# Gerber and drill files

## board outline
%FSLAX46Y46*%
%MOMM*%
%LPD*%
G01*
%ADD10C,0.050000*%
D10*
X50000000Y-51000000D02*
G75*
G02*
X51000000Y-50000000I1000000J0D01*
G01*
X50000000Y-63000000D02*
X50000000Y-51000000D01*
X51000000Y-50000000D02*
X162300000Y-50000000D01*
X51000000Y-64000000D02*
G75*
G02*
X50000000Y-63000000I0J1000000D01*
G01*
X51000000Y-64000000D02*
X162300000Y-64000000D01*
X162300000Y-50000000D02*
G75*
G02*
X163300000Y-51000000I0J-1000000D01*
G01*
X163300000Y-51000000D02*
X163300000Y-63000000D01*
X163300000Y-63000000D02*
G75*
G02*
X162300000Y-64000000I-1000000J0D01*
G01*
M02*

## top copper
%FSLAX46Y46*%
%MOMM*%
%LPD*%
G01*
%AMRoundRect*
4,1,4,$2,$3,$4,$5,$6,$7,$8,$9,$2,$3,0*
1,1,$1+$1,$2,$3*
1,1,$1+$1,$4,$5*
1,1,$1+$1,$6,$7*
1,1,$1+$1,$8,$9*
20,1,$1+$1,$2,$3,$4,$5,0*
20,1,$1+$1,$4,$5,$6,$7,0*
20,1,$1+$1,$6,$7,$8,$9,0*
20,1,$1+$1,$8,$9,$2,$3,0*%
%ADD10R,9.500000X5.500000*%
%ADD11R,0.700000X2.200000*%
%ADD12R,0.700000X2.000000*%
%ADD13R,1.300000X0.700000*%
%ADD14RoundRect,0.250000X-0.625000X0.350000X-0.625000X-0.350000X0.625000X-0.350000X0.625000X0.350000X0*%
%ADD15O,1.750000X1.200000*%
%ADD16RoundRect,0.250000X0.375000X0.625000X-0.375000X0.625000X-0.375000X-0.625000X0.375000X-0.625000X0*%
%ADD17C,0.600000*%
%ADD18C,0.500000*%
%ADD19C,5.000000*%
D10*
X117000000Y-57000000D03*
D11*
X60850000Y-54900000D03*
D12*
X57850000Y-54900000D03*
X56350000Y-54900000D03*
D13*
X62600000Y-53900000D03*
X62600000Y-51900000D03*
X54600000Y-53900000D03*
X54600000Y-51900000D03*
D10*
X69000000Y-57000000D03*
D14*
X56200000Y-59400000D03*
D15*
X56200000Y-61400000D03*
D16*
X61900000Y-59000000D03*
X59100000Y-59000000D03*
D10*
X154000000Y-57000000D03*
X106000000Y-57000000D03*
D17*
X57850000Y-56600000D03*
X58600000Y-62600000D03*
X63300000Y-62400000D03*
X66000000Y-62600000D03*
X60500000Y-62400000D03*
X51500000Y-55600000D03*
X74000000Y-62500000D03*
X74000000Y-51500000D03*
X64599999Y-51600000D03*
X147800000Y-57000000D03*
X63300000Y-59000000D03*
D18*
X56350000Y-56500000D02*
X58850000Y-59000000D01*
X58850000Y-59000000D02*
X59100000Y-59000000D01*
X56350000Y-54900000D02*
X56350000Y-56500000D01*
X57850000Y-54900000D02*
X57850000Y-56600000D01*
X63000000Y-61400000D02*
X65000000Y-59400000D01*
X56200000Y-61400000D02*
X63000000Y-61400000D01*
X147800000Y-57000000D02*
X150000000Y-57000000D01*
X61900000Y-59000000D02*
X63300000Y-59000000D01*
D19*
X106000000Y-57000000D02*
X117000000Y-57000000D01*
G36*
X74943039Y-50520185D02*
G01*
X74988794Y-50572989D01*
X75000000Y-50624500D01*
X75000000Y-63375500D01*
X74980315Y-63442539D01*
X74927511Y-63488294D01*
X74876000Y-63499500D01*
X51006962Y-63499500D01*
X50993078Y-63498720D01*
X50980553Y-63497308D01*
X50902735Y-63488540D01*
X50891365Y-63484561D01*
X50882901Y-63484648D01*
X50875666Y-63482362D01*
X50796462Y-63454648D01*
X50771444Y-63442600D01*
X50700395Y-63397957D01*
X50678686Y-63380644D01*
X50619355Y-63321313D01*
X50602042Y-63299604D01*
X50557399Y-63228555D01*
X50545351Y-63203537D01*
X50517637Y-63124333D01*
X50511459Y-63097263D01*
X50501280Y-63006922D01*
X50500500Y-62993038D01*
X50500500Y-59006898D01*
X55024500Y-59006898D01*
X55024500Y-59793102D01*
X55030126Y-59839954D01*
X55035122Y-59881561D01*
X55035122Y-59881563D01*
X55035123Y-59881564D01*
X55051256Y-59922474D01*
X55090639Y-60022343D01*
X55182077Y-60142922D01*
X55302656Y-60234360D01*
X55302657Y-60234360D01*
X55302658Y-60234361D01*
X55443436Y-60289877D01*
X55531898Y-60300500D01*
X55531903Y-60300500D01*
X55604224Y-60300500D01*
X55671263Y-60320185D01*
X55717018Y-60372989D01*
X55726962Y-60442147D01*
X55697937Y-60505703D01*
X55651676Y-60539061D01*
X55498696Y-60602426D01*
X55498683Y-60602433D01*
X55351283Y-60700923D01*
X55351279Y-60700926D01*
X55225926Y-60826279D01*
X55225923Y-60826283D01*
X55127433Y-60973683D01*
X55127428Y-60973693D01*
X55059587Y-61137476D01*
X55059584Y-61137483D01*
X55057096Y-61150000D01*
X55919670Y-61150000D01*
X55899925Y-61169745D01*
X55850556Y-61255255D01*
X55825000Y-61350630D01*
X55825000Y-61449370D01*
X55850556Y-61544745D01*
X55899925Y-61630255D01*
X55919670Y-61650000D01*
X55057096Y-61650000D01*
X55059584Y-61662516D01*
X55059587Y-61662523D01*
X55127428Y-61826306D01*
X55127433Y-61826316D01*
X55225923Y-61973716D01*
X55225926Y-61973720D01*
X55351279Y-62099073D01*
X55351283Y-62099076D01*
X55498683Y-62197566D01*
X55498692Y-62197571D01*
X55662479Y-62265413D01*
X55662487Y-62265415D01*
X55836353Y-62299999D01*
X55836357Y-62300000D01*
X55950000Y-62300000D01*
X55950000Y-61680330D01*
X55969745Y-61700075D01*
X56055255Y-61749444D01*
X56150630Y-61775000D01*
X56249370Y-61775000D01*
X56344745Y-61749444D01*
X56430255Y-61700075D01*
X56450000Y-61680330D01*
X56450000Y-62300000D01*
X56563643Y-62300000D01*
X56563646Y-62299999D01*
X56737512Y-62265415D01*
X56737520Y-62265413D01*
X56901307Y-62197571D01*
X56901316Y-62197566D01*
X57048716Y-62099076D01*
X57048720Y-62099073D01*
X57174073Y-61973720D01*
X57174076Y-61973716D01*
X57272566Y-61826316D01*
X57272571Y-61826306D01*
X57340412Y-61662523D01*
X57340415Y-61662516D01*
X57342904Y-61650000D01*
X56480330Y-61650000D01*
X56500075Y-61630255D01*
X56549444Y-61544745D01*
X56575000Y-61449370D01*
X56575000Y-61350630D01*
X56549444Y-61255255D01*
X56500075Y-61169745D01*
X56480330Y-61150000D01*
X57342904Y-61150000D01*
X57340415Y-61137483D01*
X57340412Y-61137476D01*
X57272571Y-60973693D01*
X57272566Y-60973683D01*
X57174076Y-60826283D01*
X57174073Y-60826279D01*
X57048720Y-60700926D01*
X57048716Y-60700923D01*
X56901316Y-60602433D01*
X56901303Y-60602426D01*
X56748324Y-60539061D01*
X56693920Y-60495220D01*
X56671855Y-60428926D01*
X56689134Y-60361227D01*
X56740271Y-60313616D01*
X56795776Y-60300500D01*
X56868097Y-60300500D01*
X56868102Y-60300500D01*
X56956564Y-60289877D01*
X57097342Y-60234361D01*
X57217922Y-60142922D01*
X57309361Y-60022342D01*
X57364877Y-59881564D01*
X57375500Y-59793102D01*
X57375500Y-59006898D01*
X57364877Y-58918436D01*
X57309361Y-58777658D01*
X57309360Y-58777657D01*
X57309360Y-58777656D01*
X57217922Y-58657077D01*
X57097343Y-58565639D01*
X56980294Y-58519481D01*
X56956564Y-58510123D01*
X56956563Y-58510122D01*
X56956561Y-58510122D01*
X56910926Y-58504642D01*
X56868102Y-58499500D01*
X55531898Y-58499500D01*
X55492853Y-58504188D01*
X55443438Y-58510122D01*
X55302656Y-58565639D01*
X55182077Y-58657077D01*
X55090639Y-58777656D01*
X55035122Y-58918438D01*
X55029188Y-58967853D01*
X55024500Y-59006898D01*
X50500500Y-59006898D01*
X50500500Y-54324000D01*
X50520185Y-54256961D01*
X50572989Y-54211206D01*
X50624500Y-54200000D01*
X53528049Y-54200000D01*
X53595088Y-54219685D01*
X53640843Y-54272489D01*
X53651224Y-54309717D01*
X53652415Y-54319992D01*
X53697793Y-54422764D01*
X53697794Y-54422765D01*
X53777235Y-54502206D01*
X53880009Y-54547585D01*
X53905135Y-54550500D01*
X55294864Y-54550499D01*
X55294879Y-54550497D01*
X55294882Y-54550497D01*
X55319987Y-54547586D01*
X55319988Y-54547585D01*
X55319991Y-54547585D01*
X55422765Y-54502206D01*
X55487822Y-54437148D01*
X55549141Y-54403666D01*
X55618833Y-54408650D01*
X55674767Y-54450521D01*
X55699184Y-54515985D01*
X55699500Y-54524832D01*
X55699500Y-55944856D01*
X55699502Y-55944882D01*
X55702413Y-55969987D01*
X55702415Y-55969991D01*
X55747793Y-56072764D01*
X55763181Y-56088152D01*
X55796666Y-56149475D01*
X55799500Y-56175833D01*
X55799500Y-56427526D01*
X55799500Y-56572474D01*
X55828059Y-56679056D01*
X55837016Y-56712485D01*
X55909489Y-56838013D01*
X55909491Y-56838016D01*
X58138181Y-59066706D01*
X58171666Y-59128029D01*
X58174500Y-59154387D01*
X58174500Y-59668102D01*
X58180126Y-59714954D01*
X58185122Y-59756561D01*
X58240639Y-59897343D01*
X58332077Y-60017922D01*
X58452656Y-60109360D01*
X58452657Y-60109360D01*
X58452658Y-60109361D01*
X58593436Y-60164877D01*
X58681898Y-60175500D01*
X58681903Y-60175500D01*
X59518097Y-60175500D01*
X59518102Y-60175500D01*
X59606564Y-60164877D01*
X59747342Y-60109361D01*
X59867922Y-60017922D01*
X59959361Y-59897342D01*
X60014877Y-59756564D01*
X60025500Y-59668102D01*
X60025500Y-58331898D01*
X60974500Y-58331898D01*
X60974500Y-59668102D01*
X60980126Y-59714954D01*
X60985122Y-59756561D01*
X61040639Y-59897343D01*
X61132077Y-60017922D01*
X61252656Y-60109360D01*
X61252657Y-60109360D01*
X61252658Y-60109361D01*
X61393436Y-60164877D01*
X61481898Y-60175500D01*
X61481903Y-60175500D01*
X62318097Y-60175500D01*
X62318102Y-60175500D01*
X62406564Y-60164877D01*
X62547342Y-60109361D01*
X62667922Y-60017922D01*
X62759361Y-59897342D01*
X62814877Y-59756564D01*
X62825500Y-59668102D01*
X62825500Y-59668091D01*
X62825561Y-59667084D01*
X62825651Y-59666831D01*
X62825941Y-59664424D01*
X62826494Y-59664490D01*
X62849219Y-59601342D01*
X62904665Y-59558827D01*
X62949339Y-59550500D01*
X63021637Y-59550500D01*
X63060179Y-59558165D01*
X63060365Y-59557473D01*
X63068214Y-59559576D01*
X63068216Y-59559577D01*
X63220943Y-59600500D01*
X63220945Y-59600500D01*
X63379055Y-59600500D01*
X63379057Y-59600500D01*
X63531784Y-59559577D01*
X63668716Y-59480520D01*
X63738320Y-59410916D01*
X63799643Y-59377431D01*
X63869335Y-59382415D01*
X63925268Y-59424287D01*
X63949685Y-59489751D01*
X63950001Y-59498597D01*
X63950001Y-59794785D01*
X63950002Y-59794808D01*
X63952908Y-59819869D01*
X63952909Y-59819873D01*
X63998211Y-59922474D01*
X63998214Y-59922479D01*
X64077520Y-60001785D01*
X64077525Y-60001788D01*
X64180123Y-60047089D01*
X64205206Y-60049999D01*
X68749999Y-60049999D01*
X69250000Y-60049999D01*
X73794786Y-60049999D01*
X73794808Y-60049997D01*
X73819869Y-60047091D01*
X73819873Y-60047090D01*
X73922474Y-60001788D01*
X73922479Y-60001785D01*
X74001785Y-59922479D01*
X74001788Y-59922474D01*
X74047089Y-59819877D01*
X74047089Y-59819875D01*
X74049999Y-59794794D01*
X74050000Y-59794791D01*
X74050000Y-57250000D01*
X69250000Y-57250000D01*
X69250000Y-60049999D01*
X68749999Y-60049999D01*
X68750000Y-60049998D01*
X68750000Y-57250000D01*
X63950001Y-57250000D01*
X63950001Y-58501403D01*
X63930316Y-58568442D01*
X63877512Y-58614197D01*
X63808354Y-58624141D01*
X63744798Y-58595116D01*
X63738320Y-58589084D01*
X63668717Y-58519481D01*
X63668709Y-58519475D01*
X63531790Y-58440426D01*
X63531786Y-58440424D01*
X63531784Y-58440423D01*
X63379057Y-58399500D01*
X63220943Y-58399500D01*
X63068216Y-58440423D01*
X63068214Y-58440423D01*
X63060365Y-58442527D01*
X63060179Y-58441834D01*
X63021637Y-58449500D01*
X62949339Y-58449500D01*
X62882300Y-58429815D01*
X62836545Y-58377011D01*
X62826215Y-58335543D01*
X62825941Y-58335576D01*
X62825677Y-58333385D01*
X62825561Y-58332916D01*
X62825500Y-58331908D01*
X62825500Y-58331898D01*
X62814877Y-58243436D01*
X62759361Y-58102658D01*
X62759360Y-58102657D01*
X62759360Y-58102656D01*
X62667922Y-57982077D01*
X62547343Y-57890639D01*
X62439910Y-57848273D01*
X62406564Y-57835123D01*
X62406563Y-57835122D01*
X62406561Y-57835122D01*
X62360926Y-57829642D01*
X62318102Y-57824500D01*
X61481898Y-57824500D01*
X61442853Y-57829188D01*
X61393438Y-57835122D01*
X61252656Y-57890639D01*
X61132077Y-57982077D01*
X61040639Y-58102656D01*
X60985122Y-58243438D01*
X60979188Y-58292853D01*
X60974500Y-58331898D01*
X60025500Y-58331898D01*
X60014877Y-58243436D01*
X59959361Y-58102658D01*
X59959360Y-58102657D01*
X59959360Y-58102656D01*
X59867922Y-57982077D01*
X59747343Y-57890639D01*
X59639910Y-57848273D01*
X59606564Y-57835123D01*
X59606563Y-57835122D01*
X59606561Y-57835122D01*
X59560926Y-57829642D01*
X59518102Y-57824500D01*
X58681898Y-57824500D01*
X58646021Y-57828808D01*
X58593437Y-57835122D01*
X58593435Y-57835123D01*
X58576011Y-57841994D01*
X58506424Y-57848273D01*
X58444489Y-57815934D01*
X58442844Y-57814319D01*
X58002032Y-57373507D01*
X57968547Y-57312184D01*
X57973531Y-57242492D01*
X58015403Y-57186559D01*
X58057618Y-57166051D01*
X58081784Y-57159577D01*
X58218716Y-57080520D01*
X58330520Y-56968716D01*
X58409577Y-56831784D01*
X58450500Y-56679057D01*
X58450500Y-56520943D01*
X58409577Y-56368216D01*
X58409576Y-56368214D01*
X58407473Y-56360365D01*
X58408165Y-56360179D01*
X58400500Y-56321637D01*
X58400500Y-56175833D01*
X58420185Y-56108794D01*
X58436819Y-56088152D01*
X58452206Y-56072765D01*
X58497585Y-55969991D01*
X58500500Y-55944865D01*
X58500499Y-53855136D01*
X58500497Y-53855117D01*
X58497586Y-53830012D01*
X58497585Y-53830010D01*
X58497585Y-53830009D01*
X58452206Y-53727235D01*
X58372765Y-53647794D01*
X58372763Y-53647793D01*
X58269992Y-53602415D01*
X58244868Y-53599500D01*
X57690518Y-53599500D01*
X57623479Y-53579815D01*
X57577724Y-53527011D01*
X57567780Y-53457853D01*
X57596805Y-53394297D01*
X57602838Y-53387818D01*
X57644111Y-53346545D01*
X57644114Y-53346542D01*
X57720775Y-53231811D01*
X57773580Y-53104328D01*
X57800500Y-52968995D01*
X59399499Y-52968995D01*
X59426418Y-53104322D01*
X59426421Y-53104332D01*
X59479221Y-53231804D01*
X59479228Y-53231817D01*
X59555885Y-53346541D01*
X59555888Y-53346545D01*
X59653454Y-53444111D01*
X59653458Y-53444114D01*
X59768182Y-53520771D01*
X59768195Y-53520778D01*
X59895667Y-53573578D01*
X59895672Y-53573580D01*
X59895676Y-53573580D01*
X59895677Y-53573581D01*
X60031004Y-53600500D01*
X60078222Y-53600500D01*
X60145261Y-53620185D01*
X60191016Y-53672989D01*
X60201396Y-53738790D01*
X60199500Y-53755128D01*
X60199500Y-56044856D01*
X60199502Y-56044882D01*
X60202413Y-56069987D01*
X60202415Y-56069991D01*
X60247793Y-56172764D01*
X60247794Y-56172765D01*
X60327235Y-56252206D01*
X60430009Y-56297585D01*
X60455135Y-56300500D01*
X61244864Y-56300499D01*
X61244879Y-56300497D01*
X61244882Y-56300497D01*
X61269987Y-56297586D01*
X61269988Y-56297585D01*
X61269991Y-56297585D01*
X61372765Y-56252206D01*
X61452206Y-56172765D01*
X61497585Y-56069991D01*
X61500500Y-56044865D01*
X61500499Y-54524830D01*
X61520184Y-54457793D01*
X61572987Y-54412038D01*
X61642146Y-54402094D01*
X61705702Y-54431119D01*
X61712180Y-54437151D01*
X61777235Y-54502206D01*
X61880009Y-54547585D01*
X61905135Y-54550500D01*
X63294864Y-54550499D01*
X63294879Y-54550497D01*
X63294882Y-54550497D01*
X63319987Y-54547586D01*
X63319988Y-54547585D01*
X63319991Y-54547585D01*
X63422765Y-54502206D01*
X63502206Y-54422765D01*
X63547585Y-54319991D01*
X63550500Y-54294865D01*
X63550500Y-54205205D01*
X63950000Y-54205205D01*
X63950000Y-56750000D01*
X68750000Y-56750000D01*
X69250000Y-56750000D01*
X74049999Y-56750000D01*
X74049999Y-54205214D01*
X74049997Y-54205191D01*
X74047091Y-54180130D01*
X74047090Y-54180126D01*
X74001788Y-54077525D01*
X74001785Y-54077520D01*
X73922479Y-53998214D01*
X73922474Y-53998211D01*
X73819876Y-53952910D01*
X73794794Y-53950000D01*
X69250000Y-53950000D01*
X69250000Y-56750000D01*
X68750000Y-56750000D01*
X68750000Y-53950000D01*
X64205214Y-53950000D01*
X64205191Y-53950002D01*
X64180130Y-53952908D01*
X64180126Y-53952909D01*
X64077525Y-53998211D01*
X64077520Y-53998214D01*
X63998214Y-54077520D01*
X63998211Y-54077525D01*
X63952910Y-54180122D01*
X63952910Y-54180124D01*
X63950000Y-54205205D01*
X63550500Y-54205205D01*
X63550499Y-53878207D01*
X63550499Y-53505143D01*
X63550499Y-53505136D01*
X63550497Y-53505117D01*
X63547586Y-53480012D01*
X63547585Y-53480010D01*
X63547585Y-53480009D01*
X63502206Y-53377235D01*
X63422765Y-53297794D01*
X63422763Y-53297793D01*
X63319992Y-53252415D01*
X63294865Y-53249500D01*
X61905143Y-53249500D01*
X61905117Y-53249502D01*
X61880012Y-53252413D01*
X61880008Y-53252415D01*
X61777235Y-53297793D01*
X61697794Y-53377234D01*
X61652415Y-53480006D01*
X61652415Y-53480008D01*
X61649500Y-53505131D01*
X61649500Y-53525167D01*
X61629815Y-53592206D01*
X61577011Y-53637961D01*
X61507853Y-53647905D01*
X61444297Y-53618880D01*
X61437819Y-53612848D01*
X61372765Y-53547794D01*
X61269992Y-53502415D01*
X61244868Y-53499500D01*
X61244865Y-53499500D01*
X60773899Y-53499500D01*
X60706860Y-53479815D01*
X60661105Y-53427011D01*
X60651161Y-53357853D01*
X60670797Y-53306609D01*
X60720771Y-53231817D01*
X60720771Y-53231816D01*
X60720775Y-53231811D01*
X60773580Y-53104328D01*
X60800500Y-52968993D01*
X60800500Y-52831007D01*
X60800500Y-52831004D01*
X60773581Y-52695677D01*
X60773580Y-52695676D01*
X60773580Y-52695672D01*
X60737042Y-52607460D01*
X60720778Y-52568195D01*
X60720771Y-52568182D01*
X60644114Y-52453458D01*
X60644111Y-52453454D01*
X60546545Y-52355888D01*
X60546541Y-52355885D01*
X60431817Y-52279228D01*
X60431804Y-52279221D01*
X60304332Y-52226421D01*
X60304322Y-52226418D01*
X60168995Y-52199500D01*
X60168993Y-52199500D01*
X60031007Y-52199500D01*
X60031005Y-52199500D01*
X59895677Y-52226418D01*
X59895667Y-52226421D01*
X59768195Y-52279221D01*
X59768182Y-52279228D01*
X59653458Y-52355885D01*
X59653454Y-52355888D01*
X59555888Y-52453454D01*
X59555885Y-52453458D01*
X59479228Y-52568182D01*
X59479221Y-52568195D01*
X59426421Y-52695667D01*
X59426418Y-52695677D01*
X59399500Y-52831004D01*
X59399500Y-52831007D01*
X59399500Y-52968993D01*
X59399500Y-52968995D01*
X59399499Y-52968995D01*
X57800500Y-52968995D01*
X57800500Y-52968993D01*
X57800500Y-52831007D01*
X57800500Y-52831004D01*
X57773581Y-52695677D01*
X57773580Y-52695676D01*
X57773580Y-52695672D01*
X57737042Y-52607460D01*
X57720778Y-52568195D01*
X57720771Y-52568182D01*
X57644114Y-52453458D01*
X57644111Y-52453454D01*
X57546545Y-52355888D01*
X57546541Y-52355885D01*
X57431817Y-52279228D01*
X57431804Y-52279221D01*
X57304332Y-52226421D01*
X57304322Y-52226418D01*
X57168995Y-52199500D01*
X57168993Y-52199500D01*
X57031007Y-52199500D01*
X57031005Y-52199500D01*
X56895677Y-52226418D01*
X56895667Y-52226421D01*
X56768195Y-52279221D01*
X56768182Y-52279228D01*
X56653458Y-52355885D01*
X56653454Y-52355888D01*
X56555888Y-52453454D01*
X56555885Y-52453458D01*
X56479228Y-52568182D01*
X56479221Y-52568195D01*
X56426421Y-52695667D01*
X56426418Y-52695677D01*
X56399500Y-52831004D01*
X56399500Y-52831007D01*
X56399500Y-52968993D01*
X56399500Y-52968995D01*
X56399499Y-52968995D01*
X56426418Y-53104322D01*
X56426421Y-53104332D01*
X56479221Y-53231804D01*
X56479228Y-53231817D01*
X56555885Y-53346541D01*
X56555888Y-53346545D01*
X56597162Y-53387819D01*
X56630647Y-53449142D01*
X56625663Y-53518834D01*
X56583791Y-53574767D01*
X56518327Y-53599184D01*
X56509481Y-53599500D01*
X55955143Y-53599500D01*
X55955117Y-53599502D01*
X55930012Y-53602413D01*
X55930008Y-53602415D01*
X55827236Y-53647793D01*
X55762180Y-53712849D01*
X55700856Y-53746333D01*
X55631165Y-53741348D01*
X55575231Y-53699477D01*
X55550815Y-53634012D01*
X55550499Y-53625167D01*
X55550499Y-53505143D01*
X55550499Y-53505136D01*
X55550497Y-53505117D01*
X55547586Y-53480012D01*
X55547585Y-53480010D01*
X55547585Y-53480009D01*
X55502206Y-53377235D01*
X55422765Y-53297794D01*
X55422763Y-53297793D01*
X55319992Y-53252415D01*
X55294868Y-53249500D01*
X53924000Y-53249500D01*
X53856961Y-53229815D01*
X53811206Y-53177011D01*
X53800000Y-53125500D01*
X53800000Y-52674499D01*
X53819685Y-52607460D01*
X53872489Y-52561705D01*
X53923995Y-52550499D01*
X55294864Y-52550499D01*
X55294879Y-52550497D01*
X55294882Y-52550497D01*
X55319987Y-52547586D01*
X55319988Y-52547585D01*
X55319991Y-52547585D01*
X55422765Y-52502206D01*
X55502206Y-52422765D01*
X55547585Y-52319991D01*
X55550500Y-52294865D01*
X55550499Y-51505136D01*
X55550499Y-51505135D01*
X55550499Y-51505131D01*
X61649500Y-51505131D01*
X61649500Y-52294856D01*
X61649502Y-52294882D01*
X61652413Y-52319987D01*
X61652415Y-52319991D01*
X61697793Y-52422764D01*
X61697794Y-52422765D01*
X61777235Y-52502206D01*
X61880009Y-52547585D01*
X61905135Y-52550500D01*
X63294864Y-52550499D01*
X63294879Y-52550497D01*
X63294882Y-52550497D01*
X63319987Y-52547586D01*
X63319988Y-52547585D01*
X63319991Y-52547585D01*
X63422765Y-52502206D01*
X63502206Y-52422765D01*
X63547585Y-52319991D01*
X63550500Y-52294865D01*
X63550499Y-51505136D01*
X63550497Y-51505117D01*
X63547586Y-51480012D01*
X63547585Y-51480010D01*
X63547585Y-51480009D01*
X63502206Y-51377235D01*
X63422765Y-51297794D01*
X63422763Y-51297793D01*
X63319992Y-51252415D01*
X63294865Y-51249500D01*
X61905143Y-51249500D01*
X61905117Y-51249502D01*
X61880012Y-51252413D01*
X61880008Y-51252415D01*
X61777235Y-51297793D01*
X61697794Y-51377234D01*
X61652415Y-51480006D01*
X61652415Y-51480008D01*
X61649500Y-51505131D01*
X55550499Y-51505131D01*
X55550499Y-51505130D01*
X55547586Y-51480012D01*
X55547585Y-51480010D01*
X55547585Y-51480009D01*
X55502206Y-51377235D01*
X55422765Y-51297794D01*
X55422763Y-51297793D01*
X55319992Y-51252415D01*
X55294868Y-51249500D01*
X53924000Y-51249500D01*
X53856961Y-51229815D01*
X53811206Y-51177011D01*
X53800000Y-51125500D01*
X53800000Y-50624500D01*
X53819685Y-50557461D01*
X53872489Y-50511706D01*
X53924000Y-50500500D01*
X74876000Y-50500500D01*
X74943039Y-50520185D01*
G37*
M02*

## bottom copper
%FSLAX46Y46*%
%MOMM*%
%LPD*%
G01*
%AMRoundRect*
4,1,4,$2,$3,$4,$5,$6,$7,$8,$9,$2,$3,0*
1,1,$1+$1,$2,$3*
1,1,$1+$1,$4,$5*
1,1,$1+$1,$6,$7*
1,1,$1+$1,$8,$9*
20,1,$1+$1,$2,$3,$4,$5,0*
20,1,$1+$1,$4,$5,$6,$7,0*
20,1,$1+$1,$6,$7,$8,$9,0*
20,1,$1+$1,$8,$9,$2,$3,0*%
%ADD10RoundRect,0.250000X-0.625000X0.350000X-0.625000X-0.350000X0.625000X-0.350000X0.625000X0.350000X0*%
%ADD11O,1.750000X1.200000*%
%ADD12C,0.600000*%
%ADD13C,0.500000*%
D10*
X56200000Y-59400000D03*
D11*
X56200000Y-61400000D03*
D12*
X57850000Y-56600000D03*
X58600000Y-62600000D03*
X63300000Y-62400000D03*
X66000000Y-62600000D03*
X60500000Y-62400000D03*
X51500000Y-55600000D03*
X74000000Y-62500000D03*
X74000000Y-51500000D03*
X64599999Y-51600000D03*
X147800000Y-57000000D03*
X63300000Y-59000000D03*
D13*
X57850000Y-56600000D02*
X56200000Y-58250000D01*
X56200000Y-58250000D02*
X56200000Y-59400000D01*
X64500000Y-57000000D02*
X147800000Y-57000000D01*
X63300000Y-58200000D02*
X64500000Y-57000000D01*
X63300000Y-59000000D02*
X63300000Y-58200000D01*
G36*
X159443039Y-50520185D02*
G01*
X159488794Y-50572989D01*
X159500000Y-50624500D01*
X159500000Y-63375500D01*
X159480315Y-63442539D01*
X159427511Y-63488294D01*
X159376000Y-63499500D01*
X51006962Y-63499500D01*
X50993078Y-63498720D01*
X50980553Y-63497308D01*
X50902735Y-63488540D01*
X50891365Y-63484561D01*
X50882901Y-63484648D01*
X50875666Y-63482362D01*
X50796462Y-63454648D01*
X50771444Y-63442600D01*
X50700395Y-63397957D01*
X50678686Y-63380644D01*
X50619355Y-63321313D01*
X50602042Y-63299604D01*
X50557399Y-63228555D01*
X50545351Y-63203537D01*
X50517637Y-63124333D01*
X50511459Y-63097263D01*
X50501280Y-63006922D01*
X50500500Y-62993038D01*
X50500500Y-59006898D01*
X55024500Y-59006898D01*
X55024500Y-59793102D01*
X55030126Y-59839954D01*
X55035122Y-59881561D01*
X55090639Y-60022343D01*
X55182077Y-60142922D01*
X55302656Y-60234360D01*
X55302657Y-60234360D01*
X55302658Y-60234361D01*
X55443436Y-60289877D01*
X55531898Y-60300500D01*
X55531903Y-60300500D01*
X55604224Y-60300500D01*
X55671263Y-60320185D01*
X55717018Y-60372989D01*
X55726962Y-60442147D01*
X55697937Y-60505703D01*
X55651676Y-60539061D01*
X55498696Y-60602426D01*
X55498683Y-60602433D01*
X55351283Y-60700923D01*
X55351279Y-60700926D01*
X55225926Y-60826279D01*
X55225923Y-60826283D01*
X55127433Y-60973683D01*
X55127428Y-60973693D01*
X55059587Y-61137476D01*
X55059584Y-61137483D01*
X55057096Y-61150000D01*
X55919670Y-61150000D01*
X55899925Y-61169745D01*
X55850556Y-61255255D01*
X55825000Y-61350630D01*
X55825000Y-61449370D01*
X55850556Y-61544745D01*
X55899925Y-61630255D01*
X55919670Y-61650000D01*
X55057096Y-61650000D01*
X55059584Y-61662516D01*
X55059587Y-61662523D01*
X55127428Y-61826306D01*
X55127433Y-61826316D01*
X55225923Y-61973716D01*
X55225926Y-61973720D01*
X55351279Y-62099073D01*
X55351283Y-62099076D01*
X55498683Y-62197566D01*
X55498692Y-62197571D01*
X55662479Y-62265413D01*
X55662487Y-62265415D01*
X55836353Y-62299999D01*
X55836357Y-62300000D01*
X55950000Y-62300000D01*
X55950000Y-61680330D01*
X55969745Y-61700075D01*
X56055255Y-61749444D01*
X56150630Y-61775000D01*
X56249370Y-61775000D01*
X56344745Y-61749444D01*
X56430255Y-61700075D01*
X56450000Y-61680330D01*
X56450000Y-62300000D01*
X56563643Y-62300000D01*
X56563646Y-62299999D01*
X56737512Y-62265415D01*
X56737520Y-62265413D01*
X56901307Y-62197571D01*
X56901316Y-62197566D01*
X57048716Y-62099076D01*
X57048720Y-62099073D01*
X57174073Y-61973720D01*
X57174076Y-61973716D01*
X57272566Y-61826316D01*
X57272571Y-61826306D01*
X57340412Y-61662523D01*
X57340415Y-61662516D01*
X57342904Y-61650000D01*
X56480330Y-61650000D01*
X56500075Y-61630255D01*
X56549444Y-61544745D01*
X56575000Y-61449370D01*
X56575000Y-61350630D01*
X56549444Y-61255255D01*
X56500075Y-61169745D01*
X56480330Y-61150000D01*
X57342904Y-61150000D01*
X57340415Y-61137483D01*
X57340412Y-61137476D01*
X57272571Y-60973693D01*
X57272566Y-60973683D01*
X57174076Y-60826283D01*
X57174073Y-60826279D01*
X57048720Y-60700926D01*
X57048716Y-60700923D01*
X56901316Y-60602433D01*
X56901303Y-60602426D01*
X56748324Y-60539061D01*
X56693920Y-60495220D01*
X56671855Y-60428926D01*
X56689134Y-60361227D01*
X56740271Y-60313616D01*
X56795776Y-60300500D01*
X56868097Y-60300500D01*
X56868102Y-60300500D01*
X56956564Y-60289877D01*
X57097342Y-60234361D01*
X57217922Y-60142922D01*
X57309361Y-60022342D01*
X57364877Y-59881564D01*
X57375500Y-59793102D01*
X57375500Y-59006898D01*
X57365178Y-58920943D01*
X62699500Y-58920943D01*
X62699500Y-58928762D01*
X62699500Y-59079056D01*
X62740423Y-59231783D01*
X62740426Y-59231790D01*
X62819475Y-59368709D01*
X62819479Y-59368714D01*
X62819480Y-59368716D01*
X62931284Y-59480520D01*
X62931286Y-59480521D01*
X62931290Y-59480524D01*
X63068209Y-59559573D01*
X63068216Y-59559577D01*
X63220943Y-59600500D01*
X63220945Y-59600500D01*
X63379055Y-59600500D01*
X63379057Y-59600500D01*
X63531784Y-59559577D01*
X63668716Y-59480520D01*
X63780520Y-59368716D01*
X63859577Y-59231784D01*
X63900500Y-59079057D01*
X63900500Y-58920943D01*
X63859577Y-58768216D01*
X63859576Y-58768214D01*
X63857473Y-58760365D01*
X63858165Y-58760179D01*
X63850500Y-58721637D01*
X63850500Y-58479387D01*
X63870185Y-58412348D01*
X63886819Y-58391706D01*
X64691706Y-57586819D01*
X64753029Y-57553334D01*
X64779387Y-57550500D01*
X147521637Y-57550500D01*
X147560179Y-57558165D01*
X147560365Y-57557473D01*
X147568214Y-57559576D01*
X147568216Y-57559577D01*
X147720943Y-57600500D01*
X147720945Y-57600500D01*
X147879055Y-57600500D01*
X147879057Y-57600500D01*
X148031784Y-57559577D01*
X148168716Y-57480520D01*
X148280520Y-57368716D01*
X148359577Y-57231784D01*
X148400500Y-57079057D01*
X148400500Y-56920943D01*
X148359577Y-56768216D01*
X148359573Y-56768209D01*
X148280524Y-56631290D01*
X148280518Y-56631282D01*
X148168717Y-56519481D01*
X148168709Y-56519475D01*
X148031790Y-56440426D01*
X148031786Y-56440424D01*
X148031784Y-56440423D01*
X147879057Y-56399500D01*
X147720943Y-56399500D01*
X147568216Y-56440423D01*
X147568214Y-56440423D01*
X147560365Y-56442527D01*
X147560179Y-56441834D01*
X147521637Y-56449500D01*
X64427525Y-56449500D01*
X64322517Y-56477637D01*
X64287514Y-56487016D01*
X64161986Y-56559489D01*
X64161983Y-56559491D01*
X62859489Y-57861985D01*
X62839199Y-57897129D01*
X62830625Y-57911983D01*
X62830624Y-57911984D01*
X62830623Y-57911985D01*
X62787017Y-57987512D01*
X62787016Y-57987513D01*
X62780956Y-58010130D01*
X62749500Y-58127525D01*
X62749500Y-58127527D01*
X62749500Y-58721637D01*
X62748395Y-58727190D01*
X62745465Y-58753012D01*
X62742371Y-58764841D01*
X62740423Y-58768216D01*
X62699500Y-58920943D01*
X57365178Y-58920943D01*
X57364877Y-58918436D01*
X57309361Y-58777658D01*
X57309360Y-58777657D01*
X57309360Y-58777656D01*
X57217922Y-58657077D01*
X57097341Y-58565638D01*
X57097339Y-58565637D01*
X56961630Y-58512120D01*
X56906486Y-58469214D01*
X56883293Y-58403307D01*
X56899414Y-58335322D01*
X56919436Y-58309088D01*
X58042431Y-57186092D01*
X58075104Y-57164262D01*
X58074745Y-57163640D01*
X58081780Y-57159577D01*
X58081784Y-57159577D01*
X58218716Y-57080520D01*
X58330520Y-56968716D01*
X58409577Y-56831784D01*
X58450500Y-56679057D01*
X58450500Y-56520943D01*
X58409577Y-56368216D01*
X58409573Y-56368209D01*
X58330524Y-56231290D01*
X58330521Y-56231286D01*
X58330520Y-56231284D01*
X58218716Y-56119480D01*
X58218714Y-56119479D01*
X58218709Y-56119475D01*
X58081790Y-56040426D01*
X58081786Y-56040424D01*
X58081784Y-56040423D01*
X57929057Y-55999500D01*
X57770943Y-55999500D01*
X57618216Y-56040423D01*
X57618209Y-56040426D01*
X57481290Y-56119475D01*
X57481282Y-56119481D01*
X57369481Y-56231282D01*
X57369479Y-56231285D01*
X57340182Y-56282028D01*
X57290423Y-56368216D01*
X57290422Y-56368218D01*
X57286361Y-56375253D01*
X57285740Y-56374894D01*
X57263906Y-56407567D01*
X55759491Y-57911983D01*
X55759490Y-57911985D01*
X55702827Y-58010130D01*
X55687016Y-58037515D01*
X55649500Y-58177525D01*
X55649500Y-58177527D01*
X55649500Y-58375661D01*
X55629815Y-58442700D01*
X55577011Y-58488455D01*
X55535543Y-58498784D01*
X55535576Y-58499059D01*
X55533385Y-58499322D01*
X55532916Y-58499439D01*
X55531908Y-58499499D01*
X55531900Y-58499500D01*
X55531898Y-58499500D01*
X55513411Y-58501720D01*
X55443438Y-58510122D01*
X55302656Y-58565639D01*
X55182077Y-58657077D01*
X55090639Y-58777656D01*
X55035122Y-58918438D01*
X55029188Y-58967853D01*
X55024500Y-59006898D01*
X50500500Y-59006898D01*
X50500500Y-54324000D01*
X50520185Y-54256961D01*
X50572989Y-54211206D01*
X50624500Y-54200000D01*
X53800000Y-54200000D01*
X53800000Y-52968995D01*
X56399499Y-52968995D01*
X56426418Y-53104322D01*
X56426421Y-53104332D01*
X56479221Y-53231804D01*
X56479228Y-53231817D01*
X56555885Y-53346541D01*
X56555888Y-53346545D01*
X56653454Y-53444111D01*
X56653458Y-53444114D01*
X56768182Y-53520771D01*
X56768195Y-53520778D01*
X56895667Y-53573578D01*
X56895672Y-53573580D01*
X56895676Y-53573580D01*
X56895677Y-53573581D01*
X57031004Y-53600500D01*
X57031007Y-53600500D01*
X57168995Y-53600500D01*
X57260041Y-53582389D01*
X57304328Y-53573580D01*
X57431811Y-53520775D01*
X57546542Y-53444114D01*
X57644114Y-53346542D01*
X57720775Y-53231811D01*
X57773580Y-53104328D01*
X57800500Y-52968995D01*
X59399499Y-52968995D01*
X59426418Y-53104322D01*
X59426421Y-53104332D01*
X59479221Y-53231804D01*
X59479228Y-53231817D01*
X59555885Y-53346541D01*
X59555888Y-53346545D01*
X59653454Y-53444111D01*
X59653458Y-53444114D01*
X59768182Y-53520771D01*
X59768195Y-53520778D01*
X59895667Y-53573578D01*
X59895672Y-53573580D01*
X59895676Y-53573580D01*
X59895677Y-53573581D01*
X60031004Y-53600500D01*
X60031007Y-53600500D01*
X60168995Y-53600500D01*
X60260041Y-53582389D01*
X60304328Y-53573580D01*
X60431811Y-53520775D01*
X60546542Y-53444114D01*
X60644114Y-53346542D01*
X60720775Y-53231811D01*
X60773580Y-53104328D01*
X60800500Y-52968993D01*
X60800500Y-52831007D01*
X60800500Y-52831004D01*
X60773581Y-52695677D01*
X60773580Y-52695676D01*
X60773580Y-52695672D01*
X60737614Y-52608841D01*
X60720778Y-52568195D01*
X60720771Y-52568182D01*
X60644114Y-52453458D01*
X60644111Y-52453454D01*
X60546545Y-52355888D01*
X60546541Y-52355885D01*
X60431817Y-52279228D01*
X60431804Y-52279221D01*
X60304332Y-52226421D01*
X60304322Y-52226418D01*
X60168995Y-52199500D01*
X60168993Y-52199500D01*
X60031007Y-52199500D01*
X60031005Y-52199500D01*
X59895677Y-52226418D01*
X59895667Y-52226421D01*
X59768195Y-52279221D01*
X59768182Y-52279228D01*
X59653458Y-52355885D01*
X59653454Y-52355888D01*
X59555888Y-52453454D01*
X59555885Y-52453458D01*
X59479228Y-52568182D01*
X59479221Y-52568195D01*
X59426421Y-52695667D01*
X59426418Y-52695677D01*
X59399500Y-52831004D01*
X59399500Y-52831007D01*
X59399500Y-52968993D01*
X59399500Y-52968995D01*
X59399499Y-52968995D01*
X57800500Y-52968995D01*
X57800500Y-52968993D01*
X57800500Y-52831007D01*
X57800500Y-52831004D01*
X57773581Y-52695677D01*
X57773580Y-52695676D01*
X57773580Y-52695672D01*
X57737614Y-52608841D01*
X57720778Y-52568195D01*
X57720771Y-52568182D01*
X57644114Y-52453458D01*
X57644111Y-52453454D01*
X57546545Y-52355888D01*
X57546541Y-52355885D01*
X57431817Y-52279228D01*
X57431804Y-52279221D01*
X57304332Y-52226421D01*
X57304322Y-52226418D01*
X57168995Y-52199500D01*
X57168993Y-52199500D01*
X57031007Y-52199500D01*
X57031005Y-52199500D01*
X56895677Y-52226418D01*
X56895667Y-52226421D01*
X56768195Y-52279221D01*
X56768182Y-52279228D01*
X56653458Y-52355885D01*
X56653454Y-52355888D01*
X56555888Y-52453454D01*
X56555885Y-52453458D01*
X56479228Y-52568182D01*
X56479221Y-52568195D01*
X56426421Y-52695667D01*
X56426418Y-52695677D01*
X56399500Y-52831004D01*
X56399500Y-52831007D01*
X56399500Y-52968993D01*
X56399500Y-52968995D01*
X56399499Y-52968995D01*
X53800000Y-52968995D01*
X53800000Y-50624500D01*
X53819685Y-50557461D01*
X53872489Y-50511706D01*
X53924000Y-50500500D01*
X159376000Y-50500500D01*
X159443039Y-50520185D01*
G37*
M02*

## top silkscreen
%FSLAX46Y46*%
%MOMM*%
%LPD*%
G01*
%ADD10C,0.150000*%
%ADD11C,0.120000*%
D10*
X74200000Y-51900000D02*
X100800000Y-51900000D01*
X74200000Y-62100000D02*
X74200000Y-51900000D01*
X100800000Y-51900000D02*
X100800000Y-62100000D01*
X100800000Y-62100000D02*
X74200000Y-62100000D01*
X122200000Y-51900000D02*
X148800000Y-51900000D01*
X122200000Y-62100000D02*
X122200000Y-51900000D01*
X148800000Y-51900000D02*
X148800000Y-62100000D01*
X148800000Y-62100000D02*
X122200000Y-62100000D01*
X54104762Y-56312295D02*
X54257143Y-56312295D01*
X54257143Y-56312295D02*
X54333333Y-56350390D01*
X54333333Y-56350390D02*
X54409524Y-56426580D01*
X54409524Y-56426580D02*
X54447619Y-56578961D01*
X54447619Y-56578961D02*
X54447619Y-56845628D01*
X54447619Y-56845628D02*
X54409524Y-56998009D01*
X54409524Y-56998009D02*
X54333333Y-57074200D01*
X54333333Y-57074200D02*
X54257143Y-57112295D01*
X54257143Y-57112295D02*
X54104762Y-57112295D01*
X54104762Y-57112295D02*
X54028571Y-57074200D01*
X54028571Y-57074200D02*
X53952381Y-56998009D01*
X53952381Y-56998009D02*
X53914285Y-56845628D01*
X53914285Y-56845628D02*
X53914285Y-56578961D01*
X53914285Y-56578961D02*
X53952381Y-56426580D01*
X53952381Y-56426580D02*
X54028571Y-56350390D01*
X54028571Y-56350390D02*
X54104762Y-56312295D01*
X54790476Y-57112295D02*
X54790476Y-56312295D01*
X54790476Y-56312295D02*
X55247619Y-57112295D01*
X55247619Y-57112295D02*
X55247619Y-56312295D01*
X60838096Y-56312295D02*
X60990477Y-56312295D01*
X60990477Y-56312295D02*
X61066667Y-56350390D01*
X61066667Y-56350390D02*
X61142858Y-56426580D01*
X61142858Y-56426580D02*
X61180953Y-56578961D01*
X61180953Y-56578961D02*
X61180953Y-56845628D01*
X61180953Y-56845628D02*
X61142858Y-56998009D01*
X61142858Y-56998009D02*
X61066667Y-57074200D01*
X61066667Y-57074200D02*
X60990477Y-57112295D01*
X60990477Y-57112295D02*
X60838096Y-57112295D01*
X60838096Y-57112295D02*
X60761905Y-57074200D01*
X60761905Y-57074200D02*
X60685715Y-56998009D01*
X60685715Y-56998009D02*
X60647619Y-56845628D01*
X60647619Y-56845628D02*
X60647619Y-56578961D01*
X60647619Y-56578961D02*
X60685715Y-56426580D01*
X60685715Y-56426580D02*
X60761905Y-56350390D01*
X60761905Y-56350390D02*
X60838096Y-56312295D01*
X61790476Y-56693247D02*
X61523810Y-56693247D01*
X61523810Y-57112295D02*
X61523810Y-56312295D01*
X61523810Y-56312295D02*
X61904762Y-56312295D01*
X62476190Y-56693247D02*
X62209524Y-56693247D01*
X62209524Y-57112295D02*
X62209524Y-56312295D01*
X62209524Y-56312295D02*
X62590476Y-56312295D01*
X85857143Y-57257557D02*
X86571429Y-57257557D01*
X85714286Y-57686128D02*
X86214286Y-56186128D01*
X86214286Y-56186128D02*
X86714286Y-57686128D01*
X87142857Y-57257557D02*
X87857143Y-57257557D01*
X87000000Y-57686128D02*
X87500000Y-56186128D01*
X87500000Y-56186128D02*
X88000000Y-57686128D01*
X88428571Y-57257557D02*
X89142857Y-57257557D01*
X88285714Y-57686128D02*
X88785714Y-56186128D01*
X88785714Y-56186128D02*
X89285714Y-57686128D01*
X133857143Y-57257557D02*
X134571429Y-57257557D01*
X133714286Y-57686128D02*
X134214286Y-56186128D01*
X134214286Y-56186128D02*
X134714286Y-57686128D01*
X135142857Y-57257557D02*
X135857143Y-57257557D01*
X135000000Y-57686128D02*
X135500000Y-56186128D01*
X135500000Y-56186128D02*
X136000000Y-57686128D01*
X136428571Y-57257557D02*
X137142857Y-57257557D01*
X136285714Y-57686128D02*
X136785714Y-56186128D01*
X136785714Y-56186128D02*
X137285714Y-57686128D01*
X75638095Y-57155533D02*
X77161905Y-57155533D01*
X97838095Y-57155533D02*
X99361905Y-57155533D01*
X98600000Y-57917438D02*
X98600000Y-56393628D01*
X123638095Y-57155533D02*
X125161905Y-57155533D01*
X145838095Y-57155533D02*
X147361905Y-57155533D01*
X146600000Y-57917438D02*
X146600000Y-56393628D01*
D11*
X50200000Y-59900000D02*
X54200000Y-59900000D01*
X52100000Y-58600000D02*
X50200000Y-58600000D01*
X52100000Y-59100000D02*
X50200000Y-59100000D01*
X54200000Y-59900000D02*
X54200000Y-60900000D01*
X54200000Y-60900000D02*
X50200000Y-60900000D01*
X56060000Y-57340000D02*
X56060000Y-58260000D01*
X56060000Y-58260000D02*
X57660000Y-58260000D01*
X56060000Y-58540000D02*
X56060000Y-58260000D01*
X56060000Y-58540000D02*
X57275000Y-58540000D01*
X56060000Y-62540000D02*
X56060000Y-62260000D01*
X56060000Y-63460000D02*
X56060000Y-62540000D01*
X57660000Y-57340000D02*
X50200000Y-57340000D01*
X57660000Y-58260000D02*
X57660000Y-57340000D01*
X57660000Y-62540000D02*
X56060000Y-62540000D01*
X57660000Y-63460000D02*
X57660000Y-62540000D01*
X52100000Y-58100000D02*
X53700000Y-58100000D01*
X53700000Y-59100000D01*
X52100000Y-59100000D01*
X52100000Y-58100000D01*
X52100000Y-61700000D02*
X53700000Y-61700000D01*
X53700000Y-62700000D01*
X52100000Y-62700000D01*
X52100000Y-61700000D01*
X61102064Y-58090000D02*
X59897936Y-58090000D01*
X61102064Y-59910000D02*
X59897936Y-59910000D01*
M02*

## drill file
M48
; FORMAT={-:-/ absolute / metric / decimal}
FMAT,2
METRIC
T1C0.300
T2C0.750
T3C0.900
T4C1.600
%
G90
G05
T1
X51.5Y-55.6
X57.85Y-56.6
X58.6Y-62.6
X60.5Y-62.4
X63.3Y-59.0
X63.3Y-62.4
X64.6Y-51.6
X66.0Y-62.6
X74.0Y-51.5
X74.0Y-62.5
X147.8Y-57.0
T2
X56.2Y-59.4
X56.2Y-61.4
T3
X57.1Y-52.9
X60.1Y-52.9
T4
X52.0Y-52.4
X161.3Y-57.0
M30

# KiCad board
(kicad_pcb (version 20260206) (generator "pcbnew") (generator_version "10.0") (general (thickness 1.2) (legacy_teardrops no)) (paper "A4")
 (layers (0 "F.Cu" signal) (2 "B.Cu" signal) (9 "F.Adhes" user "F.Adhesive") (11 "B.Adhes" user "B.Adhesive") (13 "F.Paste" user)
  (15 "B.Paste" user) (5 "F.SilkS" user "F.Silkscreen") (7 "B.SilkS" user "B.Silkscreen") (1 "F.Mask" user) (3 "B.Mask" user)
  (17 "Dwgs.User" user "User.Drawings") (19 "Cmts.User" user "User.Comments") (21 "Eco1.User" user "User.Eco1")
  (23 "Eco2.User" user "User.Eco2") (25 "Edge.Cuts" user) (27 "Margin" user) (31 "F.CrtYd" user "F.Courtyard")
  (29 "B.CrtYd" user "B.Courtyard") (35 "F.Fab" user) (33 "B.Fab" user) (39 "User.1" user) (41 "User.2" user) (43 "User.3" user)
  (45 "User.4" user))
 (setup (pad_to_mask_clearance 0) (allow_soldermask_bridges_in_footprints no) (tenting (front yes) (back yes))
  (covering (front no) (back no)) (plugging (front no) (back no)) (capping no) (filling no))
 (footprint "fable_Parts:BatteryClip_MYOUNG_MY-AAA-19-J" (layer "F.Cu") (at 117 57)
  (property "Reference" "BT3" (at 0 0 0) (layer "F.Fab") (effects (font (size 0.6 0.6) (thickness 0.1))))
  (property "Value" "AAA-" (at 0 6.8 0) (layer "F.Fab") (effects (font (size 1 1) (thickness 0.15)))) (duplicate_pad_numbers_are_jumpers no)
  (pad "1" smd rect (at 0 0) (size 9.5 5.5) (layers "F.Cu" "F.Mask" "F.Paste") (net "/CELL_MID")))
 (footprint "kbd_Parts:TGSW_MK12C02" (layer "F.Cu") (at 58.6 52.9 180)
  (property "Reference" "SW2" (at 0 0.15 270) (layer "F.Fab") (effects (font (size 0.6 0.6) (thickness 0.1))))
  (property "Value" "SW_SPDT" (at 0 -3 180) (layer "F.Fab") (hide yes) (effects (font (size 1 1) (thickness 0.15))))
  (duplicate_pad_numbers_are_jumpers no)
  (pad "" np_thru_hole circle (at -1.5 0 180) (size 0.9 0.9) (drill 0.9) (layers "*.Cu" "*.Mask"))
  (pad "" np_thru_hole circle (at 1.5 0 180) (size 0.9 0.9) (drill 0.9) (layers "*.Cu" "*.Mask"))
  (pad "1" smd rect (at -2.25 -2 180) (size 0.7 2.2) (layers "F.Cu" "F.Mask" "F.Paste") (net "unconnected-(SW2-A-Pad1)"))
  (pad "2" smd rect (at 0.75 -2 180) (size 0.7 2) (layers "F.Cu" "F.Mask" "F.Paste") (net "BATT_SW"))
  (pad "3" smd rect (at 2.25 -2 180) (size 0.7 2) (layers "F.Cu" "F.Mask" "F.Paste") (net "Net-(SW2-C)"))
  (pad "4" smd rect (at -4 -1 90) (size 0.7 1.3) (layers "F.Cu" "F.Mask" "F.Paste"))
  (pad "4" smd rect (at -4 1 90) (size 0.7 1.3) (layers "F.Cu" "F.Mask" "F.Paste"))
  (pad "4" smd rect (at 4 -1 90) (size 0.7 1.3) (layers "F.Cu" "F.Mask" "F.Paste"))
  (pad "4" smd rect (at 4 1 90) (size 0.7 1.3) (layers "F.Cu" "F.Mask" "F.Paste")))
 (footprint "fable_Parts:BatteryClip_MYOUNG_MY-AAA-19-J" (layer "F.Cu") (at 69 57)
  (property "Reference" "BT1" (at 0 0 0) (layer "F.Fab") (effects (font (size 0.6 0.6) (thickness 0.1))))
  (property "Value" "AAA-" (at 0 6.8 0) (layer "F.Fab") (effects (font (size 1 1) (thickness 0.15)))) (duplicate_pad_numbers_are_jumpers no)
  (pad "1" smd rect (at 0 0) (size 9.5 5.5) (layers "F.Cu" "F.Mask" "F.Paste") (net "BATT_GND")))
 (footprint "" (layer "F.Cu") (at 52 52.4)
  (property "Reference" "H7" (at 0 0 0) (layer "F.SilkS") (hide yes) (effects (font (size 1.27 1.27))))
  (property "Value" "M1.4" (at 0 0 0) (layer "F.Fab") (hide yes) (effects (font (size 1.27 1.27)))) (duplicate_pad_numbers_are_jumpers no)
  (pad "" np_thru_hole circle (at 0 0) (size 1.6 1.6) (drill 1.6) (layers "*.Cu")))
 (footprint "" (layer "F.Cu") (at 161.3 57)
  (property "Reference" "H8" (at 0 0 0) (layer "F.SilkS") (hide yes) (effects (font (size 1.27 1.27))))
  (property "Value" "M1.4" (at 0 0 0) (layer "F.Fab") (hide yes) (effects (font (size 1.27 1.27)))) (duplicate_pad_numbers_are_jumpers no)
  (pad "" np_thru_hole circle (at 0 0) (size 1.6 1.6) (drill 1.6) (layers "*.Cu")))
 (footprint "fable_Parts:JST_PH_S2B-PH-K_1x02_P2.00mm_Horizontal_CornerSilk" (layer "F.Cu") (at 56.2 59.4 -90)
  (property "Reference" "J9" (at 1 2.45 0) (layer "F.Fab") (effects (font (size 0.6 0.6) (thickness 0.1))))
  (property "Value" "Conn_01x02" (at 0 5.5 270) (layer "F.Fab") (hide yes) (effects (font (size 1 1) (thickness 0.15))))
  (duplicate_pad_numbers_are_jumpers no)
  (fp_line (start 0.5 6) (end 0.5 2) (stroke (width 0.12) (type solid)) (layer "F.SilkS"))
  (fp_line (start -0.8 4.1) (end -0.8 6) (stroke (width 0.12) (type solid)) (layer "F.SilkS"))
  (fp_line (start -0.3 4.1) (end -0.3 6) (stroke (width 0.12) (type solid)) (layer "F.SilkS"))
  (fp_line (start 0.5 2) (end 1.5 2) (stroke (width 0.12) (type solid)) (layer "F.SilkS"))
  (fp_line (start 1.5 2) (end 1.5 6) (stroke (width 0.12) (type solid)) (layer "F.SilkS"))
  (fp_line (start -2.06 0.14) (end -1.14 0.14) (stroke (width 0.12) (type solid)) (layer "F.SilkS"))
  (fp_line (start -1.14 0.14) (end -1.14 -1.46) (stroke (width 0.12) (type solid)) (layer "F.SilkS"))
  (fp_line (start -0.86 0.14) (end -1.14 0.14) (stroke (width 0.12) (type solid)) (layer "F.SilkS"))
  (fp_line (start -0.86 0.14) (end -0.86 -1.075) (stroke (width 0.12) (type solid)) (layer "F.SilkS"))
  (fp_line (start 3.14 0.14) (end 2.86 0.14) (stroke (width 0.12) (type solid)) (layer "F.SilkS"))
  (fp_line (start 4.06 0.14) (end 3.14 0.14) (stroke (width 0.12) (type solid)) (layer "F.SilkS"))
  (fp_line (start -2.06 -1.46) (end -2.06 6) (stroke (width 0.12) (type solid)) (layer "F.SilkS"))
  (fp_line (start -1.14 -1.46) (end -2.06 -1.46) (stroke (width 0.12) (type solid)) (layer "F.SilkS"))
  (fp_line (start 3.14 -1.46) (end 3.14 0.14) (stroke (width 0.12) (type solid)) (layer "F.SilkS"))
  (fp_line (start 4.06 -1.46) (end 3.14 -1.46) (stroke (width 0.12) (type solid)) (layer "F.SilkS"))
  (fp_rect (start -1.3 2.5) (end -0.3 4.1) (stroke (width 0.12) (type solid)) (fill no) (layer "F.SilkS"))
  (fp_rect (start 2.3 2.5) (end 3.3 4.1) (stroke (width 0.12) (type solid)) (fill no) (layer "F.SilkS"))
  (pad "1" thru_hole roundrect (at 0 0 270) (size 1.2 1.75) (drill 0.75) (layers "*.Cu" "*.Mask") (remove_unused_layers no)
   (roundrect_rratio 0.208333) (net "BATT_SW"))
  (pad "2" thru_hole oval (at 2 0 270) (size 1.2 1.75) (drill 0.75) (layers "*.Cu" "*.Mask") (remove_unused_layers no) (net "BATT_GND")))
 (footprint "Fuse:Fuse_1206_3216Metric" (layer "F.Cu") (at 60.5 59 180)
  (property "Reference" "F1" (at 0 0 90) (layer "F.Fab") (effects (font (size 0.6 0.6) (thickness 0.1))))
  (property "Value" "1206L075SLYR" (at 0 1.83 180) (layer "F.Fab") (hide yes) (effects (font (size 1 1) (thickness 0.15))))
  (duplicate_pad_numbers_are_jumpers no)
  (fp_line (start -0.602064 0.91) (end 0.602064 0.91) (stroke (width 0.12) (type solid)) (layer "F.SilkS"))
  (fp_line (start -0.602064 -0.91) (end 0.602064 -0.91) (stroke (width 0.12) (type solid)) (layer "F.SilkS"))
  (pad "1" smd roundrect (at -1.4 0 180) (size 1.25 1.75) (layers "F.Cu" "F.Mask" "F.Paste") (roundrect_rratio 0.2) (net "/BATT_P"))
  (pad "2" smd roundrect (at 1.4 0 180) (size 1.25 1.75) (layers "F.Cu" "F.Mask" "F.Paste") (roundrect_rratio 0.2) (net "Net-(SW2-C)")))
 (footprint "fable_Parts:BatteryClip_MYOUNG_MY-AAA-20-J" (layer "F.Cu") (at 154 57 180)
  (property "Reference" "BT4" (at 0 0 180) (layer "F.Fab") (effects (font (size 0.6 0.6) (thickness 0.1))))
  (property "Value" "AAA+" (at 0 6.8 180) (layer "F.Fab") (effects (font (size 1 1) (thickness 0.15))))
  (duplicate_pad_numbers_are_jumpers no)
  (pad "1" smd rect (at 0 0 180) (size 9.5 5.5) (layers "F.Cu" "F.Mask" "F.Paste") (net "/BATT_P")))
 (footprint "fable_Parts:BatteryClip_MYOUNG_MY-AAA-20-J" (layer "F.Cu") (at 106 57 180)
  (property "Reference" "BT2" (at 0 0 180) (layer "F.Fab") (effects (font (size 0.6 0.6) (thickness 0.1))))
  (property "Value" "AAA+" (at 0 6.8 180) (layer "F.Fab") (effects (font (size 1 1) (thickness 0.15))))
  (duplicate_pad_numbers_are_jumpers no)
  (pad "1" smd rect (at 0 0 180) (size 9.5 5.5) (layers "F.Cu" "F.Mask" "F.Paste") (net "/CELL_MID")))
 (gr_line (start 74.2 51.9) (end 100.8 51.9) (stroke (width 0.15) (type default)) (layer "F.SilkS"))
 (gr_line (start 74.2 62.1) (end 74.2 51.9) (stroke (width 0.15) (type default)) (layer "F.SilkS"))
 (gr_line (start 100.8 51.9) (end 100.8 62.1) (stroke (width 0.15) (type default)) (layer "F.SilkS"))
 (gr_line (start 100.8 62.1) (end 74.2 62.1) (stroke (width 0.15) (type default)) (layer "F.SilkS"))
 (gr_line (start 122.2 51.9) (end 148.8 51.9) (stroke (width 0.15) (type default)) (layer "F.SilkS"))
 (gr_line (start 122.2 62.1) (end 122.2 51.9) (stroke (width 0.15) (type default)) (layer "F.SilkS"))
 (gr_line (start 148.8 51.9) (end 148.8 62.1) (stroke (width 0.15) (type default)) (layer "F.SilkS"))
 (gr_line (start 148.8 62.1) (end 122.2 62.1) (stroke (width 0.15) (type default)) (layer "F.SilkS"))
 (gr_arc (start 50 51) (mid 50.292893 50.292893) (end 51 50) (stroke (width 0.05) (type default)) (layer "Edge.Cuts"))
 (gr_line (start 50 63) (end 50 51) (stroke (width 0.05) (type default)) (layer "Edge.Cuts"))
 (gr_line (start 51 50) (end 162.3 50) (stroke (width 0.05) (type default)) (layer "Edge.Cuts"))
 (gr_arc (start 51 64) (mid 50.292893 63.707106) (end 50 63) (stroke (width 0.05) (type default)) (layer "Edge.Cuts"))
 (gr_line (start 51 64) (end 162.3 64) (stroke (width 0.05) (type default)) (layer "Edge.Cuts"))
 (gr_arc (start 162.3 50) (mid 163.007106 50.292893) (end 163.3 51) (stroke (width 0.05) (type default)) (layer "Edge.Cuts"))
 (gr_line (start 163.3 51) (end 163.3 63) (stroke (width 0.05) (type default)) (layer "Edge.Cuts"))
 (gr_arc (start 163.3 63) (mid 163.007106 63.707106) (end 162.3 64) (stroke (width 0.05) (type default)) (layer "Edge.Cuts"))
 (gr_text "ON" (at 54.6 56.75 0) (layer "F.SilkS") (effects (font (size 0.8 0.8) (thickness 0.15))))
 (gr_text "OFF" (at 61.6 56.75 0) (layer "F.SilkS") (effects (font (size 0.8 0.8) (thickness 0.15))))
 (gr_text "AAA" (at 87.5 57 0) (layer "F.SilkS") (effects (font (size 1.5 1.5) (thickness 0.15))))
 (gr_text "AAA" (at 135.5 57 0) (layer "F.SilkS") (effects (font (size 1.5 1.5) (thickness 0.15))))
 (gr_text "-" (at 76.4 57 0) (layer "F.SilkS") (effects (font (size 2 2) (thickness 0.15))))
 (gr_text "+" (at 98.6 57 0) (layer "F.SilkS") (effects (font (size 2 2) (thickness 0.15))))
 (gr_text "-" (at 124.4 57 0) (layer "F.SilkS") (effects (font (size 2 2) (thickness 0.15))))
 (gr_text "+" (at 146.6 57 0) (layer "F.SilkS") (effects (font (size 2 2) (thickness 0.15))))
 (segment (start 56.35 56.5) (end 58.85 59) (width 0.5) (layer "F.Cu") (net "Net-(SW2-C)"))
 (segment (start 58.85 59) (end 59.1 59) (width 0.5) (layer "F.Cu") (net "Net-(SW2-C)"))
 (segment (start 56.35 54.9) (end 56.35 56.5) (width 0.5) (layer "F.Cu") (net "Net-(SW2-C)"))
 (segment (start 57.85 54.9) (end 57.85 56.6) (width 0.5) (layer "F.Cu") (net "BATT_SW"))
 (via (at 57.85 56.6) (size 0.6) (drill 0.3) (layers "F.Cu" "B.Cu") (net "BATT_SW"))
 (segment (start 57.85 56.6) (end 56.2 58.25) (width 0.5) (layer "B.Cu") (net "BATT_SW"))
 (segment (start 56.2 58.25) (end 56.2 59.4) (width 0.5) (layer "B.Cu") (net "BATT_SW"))
 (segment (start 63 61.4) (end 65 59.4) (width 0.5) (layer "F.Cu") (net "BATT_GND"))
 (segment (start 56.2 61.4) (end 63 61.4) (width 0.5) (layer "F.Cu") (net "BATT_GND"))
 (via (at 58.6 62.6) (size 0.6) (drill 0.3) (layers "F.Cu" "B.Cu") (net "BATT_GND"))
 (via (at 63.3 62.4) (size 0.6) (drill 0.3) (layers "F.Cu" "B.Cu") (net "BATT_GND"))
 (via (at 66 62.6) (size 0.6) (drill 0.3) (layers "F.Cu" "B.Cu") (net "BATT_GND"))
 (via (at 60.5 62.4) (size 0.6) (drill 0.3) (layers "F.Cu" "B.Cu") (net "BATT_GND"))
 (via (at 51.5 55.6) (size 0.6) (drill 0.3) (layers "F.Cu" "B.Cu") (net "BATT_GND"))
 (via (at 74 62.5) (size 0.6) (drill 0.3) (layers "F.Cu" "B.Cu") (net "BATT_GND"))
 (via (at 74 51.5) (size 0.6) (drill 0.3) (layers "F.Cu" "B.Cu") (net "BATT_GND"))
 (via (at 64.599999 51.6) (size 0.6) (drill 0.3) (layers "F.Cu" "B.Cu") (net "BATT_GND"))
 (segment (start 147.8 57) (end 150 57) (width 0.5) (layer "F.Cu") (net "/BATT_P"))
 (segment (start 61.9 59) (end 63.3 59) (width 0.5) (layer "F.Cu") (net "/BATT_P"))
 (via (at 147.8 57) (size 0.6) (drill 0.3) (layers "F.Cu" "B.Cu") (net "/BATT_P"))
 (via (at 63.3 59) (size 0.6) (drill 0.3) (layers "F.Cu" "B.Cu") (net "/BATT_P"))
 (segment (start 64.5 57) (end 147.8 57) (width 0.5) (layer "B.Cu") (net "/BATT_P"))
 (segment (start 63.3 58.2) (end 64.5 57) (width 0.5) (layer "B.Cu") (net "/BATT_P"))
 (segment (start 63.3 59) (end 63.3 58.2) (width 0.5) (layer "B.Cu") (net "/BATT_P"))
 (segment (start 106 57) (end 117 57) (width 5) (layer "F.Cu") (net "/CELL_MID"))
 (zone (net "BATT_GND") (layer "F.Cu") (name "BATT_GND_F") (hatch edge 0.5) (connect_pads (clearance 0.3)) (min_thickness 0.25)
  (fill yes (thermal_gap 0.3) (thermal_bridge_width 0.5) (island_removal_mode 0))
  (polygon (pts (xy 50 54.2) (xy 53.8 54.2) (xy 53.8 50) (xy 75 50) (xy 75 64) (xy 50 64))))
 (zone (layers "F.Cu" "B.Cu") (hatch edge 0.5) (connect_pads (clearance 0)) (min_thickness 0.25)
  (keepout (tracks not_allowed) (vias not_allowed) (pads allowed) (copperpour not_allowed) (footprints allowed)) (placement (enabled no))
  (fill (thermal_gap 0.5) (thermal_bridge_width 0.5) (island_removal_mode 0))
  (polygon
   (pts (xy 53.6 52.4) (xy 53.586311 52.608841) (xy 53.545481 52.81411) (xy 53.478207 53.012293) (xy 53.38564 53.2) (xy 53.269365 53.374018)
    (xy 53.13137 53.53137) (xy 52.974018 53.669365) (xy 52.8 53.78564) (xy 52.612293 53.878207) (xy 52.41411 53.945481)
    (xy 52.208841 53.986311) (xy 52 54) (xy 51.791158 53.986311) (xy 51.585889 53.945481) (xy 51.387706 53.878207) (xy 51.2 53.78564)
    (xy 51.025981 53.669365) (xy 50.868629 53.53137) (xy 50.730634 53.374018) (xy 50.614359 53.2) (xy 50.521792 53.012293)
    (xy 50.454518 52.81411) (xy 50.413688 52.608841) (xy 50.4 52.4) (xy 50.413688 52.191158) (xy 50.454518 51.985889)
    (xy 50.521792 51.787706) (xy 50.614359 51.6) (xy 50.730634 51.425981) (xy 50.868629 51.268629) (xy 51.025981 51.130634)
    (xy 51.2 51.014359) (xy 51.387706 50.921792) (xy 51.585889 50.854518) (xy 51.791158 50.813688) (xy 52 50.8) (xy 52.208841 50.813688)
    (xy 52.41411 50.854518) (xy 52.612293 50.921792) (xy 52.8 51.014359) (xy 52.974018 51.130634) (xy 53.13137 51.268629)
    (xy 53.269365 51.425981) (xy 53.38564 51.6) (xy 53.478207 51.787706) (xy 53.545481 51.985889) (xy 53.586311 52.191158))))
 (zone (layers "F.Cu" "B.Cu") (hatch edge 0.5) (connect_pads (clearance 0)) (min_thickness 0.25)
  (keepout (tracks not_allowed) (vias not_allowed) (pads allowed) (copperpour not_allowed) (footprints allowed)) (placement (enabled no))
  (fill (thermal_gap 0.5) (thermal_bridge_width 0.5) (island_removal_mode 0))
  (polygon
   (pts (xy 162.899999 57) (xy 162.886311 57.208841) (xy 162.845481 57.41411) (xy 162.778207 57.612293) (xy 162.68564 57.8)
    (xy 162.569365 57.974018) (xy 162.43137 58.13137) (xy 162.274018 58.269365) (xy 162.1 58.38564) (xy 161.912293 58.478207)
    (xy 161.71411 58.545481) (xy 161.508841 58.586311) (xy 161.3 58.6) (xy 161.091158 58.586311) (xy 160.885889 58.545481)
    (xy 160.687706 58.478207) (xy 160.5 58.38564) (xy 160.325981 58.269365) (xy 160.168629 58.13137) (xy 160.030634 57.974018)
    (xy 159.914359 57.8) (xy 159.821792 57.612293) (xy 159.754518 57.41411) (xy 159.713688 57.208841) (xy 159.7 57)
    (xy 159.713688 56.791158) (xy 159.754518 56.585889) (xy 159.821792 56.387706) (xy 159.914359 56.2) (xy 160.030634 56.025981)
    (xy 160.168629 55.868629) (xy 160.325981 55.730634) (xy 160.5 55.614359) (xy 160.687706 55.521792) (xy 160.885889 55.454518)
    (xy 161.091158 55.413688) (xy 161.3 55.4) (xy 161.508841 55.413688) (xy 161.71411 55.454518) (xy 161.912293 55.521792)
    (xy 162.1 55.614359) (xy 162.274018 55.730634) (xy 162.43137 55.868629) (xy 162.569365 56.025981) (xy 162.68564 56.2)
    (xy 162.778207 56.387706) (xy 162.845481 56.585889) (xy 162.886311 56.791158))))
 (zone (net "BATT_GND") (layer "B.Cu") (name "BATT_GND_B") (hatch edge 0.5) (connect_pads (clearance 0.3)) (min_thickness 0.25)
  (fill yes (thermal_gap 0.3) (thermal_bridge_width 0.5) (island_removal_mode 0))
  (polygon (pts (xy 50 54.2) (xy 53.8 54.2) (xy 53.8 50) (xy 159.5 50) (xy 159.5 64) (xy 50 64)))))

